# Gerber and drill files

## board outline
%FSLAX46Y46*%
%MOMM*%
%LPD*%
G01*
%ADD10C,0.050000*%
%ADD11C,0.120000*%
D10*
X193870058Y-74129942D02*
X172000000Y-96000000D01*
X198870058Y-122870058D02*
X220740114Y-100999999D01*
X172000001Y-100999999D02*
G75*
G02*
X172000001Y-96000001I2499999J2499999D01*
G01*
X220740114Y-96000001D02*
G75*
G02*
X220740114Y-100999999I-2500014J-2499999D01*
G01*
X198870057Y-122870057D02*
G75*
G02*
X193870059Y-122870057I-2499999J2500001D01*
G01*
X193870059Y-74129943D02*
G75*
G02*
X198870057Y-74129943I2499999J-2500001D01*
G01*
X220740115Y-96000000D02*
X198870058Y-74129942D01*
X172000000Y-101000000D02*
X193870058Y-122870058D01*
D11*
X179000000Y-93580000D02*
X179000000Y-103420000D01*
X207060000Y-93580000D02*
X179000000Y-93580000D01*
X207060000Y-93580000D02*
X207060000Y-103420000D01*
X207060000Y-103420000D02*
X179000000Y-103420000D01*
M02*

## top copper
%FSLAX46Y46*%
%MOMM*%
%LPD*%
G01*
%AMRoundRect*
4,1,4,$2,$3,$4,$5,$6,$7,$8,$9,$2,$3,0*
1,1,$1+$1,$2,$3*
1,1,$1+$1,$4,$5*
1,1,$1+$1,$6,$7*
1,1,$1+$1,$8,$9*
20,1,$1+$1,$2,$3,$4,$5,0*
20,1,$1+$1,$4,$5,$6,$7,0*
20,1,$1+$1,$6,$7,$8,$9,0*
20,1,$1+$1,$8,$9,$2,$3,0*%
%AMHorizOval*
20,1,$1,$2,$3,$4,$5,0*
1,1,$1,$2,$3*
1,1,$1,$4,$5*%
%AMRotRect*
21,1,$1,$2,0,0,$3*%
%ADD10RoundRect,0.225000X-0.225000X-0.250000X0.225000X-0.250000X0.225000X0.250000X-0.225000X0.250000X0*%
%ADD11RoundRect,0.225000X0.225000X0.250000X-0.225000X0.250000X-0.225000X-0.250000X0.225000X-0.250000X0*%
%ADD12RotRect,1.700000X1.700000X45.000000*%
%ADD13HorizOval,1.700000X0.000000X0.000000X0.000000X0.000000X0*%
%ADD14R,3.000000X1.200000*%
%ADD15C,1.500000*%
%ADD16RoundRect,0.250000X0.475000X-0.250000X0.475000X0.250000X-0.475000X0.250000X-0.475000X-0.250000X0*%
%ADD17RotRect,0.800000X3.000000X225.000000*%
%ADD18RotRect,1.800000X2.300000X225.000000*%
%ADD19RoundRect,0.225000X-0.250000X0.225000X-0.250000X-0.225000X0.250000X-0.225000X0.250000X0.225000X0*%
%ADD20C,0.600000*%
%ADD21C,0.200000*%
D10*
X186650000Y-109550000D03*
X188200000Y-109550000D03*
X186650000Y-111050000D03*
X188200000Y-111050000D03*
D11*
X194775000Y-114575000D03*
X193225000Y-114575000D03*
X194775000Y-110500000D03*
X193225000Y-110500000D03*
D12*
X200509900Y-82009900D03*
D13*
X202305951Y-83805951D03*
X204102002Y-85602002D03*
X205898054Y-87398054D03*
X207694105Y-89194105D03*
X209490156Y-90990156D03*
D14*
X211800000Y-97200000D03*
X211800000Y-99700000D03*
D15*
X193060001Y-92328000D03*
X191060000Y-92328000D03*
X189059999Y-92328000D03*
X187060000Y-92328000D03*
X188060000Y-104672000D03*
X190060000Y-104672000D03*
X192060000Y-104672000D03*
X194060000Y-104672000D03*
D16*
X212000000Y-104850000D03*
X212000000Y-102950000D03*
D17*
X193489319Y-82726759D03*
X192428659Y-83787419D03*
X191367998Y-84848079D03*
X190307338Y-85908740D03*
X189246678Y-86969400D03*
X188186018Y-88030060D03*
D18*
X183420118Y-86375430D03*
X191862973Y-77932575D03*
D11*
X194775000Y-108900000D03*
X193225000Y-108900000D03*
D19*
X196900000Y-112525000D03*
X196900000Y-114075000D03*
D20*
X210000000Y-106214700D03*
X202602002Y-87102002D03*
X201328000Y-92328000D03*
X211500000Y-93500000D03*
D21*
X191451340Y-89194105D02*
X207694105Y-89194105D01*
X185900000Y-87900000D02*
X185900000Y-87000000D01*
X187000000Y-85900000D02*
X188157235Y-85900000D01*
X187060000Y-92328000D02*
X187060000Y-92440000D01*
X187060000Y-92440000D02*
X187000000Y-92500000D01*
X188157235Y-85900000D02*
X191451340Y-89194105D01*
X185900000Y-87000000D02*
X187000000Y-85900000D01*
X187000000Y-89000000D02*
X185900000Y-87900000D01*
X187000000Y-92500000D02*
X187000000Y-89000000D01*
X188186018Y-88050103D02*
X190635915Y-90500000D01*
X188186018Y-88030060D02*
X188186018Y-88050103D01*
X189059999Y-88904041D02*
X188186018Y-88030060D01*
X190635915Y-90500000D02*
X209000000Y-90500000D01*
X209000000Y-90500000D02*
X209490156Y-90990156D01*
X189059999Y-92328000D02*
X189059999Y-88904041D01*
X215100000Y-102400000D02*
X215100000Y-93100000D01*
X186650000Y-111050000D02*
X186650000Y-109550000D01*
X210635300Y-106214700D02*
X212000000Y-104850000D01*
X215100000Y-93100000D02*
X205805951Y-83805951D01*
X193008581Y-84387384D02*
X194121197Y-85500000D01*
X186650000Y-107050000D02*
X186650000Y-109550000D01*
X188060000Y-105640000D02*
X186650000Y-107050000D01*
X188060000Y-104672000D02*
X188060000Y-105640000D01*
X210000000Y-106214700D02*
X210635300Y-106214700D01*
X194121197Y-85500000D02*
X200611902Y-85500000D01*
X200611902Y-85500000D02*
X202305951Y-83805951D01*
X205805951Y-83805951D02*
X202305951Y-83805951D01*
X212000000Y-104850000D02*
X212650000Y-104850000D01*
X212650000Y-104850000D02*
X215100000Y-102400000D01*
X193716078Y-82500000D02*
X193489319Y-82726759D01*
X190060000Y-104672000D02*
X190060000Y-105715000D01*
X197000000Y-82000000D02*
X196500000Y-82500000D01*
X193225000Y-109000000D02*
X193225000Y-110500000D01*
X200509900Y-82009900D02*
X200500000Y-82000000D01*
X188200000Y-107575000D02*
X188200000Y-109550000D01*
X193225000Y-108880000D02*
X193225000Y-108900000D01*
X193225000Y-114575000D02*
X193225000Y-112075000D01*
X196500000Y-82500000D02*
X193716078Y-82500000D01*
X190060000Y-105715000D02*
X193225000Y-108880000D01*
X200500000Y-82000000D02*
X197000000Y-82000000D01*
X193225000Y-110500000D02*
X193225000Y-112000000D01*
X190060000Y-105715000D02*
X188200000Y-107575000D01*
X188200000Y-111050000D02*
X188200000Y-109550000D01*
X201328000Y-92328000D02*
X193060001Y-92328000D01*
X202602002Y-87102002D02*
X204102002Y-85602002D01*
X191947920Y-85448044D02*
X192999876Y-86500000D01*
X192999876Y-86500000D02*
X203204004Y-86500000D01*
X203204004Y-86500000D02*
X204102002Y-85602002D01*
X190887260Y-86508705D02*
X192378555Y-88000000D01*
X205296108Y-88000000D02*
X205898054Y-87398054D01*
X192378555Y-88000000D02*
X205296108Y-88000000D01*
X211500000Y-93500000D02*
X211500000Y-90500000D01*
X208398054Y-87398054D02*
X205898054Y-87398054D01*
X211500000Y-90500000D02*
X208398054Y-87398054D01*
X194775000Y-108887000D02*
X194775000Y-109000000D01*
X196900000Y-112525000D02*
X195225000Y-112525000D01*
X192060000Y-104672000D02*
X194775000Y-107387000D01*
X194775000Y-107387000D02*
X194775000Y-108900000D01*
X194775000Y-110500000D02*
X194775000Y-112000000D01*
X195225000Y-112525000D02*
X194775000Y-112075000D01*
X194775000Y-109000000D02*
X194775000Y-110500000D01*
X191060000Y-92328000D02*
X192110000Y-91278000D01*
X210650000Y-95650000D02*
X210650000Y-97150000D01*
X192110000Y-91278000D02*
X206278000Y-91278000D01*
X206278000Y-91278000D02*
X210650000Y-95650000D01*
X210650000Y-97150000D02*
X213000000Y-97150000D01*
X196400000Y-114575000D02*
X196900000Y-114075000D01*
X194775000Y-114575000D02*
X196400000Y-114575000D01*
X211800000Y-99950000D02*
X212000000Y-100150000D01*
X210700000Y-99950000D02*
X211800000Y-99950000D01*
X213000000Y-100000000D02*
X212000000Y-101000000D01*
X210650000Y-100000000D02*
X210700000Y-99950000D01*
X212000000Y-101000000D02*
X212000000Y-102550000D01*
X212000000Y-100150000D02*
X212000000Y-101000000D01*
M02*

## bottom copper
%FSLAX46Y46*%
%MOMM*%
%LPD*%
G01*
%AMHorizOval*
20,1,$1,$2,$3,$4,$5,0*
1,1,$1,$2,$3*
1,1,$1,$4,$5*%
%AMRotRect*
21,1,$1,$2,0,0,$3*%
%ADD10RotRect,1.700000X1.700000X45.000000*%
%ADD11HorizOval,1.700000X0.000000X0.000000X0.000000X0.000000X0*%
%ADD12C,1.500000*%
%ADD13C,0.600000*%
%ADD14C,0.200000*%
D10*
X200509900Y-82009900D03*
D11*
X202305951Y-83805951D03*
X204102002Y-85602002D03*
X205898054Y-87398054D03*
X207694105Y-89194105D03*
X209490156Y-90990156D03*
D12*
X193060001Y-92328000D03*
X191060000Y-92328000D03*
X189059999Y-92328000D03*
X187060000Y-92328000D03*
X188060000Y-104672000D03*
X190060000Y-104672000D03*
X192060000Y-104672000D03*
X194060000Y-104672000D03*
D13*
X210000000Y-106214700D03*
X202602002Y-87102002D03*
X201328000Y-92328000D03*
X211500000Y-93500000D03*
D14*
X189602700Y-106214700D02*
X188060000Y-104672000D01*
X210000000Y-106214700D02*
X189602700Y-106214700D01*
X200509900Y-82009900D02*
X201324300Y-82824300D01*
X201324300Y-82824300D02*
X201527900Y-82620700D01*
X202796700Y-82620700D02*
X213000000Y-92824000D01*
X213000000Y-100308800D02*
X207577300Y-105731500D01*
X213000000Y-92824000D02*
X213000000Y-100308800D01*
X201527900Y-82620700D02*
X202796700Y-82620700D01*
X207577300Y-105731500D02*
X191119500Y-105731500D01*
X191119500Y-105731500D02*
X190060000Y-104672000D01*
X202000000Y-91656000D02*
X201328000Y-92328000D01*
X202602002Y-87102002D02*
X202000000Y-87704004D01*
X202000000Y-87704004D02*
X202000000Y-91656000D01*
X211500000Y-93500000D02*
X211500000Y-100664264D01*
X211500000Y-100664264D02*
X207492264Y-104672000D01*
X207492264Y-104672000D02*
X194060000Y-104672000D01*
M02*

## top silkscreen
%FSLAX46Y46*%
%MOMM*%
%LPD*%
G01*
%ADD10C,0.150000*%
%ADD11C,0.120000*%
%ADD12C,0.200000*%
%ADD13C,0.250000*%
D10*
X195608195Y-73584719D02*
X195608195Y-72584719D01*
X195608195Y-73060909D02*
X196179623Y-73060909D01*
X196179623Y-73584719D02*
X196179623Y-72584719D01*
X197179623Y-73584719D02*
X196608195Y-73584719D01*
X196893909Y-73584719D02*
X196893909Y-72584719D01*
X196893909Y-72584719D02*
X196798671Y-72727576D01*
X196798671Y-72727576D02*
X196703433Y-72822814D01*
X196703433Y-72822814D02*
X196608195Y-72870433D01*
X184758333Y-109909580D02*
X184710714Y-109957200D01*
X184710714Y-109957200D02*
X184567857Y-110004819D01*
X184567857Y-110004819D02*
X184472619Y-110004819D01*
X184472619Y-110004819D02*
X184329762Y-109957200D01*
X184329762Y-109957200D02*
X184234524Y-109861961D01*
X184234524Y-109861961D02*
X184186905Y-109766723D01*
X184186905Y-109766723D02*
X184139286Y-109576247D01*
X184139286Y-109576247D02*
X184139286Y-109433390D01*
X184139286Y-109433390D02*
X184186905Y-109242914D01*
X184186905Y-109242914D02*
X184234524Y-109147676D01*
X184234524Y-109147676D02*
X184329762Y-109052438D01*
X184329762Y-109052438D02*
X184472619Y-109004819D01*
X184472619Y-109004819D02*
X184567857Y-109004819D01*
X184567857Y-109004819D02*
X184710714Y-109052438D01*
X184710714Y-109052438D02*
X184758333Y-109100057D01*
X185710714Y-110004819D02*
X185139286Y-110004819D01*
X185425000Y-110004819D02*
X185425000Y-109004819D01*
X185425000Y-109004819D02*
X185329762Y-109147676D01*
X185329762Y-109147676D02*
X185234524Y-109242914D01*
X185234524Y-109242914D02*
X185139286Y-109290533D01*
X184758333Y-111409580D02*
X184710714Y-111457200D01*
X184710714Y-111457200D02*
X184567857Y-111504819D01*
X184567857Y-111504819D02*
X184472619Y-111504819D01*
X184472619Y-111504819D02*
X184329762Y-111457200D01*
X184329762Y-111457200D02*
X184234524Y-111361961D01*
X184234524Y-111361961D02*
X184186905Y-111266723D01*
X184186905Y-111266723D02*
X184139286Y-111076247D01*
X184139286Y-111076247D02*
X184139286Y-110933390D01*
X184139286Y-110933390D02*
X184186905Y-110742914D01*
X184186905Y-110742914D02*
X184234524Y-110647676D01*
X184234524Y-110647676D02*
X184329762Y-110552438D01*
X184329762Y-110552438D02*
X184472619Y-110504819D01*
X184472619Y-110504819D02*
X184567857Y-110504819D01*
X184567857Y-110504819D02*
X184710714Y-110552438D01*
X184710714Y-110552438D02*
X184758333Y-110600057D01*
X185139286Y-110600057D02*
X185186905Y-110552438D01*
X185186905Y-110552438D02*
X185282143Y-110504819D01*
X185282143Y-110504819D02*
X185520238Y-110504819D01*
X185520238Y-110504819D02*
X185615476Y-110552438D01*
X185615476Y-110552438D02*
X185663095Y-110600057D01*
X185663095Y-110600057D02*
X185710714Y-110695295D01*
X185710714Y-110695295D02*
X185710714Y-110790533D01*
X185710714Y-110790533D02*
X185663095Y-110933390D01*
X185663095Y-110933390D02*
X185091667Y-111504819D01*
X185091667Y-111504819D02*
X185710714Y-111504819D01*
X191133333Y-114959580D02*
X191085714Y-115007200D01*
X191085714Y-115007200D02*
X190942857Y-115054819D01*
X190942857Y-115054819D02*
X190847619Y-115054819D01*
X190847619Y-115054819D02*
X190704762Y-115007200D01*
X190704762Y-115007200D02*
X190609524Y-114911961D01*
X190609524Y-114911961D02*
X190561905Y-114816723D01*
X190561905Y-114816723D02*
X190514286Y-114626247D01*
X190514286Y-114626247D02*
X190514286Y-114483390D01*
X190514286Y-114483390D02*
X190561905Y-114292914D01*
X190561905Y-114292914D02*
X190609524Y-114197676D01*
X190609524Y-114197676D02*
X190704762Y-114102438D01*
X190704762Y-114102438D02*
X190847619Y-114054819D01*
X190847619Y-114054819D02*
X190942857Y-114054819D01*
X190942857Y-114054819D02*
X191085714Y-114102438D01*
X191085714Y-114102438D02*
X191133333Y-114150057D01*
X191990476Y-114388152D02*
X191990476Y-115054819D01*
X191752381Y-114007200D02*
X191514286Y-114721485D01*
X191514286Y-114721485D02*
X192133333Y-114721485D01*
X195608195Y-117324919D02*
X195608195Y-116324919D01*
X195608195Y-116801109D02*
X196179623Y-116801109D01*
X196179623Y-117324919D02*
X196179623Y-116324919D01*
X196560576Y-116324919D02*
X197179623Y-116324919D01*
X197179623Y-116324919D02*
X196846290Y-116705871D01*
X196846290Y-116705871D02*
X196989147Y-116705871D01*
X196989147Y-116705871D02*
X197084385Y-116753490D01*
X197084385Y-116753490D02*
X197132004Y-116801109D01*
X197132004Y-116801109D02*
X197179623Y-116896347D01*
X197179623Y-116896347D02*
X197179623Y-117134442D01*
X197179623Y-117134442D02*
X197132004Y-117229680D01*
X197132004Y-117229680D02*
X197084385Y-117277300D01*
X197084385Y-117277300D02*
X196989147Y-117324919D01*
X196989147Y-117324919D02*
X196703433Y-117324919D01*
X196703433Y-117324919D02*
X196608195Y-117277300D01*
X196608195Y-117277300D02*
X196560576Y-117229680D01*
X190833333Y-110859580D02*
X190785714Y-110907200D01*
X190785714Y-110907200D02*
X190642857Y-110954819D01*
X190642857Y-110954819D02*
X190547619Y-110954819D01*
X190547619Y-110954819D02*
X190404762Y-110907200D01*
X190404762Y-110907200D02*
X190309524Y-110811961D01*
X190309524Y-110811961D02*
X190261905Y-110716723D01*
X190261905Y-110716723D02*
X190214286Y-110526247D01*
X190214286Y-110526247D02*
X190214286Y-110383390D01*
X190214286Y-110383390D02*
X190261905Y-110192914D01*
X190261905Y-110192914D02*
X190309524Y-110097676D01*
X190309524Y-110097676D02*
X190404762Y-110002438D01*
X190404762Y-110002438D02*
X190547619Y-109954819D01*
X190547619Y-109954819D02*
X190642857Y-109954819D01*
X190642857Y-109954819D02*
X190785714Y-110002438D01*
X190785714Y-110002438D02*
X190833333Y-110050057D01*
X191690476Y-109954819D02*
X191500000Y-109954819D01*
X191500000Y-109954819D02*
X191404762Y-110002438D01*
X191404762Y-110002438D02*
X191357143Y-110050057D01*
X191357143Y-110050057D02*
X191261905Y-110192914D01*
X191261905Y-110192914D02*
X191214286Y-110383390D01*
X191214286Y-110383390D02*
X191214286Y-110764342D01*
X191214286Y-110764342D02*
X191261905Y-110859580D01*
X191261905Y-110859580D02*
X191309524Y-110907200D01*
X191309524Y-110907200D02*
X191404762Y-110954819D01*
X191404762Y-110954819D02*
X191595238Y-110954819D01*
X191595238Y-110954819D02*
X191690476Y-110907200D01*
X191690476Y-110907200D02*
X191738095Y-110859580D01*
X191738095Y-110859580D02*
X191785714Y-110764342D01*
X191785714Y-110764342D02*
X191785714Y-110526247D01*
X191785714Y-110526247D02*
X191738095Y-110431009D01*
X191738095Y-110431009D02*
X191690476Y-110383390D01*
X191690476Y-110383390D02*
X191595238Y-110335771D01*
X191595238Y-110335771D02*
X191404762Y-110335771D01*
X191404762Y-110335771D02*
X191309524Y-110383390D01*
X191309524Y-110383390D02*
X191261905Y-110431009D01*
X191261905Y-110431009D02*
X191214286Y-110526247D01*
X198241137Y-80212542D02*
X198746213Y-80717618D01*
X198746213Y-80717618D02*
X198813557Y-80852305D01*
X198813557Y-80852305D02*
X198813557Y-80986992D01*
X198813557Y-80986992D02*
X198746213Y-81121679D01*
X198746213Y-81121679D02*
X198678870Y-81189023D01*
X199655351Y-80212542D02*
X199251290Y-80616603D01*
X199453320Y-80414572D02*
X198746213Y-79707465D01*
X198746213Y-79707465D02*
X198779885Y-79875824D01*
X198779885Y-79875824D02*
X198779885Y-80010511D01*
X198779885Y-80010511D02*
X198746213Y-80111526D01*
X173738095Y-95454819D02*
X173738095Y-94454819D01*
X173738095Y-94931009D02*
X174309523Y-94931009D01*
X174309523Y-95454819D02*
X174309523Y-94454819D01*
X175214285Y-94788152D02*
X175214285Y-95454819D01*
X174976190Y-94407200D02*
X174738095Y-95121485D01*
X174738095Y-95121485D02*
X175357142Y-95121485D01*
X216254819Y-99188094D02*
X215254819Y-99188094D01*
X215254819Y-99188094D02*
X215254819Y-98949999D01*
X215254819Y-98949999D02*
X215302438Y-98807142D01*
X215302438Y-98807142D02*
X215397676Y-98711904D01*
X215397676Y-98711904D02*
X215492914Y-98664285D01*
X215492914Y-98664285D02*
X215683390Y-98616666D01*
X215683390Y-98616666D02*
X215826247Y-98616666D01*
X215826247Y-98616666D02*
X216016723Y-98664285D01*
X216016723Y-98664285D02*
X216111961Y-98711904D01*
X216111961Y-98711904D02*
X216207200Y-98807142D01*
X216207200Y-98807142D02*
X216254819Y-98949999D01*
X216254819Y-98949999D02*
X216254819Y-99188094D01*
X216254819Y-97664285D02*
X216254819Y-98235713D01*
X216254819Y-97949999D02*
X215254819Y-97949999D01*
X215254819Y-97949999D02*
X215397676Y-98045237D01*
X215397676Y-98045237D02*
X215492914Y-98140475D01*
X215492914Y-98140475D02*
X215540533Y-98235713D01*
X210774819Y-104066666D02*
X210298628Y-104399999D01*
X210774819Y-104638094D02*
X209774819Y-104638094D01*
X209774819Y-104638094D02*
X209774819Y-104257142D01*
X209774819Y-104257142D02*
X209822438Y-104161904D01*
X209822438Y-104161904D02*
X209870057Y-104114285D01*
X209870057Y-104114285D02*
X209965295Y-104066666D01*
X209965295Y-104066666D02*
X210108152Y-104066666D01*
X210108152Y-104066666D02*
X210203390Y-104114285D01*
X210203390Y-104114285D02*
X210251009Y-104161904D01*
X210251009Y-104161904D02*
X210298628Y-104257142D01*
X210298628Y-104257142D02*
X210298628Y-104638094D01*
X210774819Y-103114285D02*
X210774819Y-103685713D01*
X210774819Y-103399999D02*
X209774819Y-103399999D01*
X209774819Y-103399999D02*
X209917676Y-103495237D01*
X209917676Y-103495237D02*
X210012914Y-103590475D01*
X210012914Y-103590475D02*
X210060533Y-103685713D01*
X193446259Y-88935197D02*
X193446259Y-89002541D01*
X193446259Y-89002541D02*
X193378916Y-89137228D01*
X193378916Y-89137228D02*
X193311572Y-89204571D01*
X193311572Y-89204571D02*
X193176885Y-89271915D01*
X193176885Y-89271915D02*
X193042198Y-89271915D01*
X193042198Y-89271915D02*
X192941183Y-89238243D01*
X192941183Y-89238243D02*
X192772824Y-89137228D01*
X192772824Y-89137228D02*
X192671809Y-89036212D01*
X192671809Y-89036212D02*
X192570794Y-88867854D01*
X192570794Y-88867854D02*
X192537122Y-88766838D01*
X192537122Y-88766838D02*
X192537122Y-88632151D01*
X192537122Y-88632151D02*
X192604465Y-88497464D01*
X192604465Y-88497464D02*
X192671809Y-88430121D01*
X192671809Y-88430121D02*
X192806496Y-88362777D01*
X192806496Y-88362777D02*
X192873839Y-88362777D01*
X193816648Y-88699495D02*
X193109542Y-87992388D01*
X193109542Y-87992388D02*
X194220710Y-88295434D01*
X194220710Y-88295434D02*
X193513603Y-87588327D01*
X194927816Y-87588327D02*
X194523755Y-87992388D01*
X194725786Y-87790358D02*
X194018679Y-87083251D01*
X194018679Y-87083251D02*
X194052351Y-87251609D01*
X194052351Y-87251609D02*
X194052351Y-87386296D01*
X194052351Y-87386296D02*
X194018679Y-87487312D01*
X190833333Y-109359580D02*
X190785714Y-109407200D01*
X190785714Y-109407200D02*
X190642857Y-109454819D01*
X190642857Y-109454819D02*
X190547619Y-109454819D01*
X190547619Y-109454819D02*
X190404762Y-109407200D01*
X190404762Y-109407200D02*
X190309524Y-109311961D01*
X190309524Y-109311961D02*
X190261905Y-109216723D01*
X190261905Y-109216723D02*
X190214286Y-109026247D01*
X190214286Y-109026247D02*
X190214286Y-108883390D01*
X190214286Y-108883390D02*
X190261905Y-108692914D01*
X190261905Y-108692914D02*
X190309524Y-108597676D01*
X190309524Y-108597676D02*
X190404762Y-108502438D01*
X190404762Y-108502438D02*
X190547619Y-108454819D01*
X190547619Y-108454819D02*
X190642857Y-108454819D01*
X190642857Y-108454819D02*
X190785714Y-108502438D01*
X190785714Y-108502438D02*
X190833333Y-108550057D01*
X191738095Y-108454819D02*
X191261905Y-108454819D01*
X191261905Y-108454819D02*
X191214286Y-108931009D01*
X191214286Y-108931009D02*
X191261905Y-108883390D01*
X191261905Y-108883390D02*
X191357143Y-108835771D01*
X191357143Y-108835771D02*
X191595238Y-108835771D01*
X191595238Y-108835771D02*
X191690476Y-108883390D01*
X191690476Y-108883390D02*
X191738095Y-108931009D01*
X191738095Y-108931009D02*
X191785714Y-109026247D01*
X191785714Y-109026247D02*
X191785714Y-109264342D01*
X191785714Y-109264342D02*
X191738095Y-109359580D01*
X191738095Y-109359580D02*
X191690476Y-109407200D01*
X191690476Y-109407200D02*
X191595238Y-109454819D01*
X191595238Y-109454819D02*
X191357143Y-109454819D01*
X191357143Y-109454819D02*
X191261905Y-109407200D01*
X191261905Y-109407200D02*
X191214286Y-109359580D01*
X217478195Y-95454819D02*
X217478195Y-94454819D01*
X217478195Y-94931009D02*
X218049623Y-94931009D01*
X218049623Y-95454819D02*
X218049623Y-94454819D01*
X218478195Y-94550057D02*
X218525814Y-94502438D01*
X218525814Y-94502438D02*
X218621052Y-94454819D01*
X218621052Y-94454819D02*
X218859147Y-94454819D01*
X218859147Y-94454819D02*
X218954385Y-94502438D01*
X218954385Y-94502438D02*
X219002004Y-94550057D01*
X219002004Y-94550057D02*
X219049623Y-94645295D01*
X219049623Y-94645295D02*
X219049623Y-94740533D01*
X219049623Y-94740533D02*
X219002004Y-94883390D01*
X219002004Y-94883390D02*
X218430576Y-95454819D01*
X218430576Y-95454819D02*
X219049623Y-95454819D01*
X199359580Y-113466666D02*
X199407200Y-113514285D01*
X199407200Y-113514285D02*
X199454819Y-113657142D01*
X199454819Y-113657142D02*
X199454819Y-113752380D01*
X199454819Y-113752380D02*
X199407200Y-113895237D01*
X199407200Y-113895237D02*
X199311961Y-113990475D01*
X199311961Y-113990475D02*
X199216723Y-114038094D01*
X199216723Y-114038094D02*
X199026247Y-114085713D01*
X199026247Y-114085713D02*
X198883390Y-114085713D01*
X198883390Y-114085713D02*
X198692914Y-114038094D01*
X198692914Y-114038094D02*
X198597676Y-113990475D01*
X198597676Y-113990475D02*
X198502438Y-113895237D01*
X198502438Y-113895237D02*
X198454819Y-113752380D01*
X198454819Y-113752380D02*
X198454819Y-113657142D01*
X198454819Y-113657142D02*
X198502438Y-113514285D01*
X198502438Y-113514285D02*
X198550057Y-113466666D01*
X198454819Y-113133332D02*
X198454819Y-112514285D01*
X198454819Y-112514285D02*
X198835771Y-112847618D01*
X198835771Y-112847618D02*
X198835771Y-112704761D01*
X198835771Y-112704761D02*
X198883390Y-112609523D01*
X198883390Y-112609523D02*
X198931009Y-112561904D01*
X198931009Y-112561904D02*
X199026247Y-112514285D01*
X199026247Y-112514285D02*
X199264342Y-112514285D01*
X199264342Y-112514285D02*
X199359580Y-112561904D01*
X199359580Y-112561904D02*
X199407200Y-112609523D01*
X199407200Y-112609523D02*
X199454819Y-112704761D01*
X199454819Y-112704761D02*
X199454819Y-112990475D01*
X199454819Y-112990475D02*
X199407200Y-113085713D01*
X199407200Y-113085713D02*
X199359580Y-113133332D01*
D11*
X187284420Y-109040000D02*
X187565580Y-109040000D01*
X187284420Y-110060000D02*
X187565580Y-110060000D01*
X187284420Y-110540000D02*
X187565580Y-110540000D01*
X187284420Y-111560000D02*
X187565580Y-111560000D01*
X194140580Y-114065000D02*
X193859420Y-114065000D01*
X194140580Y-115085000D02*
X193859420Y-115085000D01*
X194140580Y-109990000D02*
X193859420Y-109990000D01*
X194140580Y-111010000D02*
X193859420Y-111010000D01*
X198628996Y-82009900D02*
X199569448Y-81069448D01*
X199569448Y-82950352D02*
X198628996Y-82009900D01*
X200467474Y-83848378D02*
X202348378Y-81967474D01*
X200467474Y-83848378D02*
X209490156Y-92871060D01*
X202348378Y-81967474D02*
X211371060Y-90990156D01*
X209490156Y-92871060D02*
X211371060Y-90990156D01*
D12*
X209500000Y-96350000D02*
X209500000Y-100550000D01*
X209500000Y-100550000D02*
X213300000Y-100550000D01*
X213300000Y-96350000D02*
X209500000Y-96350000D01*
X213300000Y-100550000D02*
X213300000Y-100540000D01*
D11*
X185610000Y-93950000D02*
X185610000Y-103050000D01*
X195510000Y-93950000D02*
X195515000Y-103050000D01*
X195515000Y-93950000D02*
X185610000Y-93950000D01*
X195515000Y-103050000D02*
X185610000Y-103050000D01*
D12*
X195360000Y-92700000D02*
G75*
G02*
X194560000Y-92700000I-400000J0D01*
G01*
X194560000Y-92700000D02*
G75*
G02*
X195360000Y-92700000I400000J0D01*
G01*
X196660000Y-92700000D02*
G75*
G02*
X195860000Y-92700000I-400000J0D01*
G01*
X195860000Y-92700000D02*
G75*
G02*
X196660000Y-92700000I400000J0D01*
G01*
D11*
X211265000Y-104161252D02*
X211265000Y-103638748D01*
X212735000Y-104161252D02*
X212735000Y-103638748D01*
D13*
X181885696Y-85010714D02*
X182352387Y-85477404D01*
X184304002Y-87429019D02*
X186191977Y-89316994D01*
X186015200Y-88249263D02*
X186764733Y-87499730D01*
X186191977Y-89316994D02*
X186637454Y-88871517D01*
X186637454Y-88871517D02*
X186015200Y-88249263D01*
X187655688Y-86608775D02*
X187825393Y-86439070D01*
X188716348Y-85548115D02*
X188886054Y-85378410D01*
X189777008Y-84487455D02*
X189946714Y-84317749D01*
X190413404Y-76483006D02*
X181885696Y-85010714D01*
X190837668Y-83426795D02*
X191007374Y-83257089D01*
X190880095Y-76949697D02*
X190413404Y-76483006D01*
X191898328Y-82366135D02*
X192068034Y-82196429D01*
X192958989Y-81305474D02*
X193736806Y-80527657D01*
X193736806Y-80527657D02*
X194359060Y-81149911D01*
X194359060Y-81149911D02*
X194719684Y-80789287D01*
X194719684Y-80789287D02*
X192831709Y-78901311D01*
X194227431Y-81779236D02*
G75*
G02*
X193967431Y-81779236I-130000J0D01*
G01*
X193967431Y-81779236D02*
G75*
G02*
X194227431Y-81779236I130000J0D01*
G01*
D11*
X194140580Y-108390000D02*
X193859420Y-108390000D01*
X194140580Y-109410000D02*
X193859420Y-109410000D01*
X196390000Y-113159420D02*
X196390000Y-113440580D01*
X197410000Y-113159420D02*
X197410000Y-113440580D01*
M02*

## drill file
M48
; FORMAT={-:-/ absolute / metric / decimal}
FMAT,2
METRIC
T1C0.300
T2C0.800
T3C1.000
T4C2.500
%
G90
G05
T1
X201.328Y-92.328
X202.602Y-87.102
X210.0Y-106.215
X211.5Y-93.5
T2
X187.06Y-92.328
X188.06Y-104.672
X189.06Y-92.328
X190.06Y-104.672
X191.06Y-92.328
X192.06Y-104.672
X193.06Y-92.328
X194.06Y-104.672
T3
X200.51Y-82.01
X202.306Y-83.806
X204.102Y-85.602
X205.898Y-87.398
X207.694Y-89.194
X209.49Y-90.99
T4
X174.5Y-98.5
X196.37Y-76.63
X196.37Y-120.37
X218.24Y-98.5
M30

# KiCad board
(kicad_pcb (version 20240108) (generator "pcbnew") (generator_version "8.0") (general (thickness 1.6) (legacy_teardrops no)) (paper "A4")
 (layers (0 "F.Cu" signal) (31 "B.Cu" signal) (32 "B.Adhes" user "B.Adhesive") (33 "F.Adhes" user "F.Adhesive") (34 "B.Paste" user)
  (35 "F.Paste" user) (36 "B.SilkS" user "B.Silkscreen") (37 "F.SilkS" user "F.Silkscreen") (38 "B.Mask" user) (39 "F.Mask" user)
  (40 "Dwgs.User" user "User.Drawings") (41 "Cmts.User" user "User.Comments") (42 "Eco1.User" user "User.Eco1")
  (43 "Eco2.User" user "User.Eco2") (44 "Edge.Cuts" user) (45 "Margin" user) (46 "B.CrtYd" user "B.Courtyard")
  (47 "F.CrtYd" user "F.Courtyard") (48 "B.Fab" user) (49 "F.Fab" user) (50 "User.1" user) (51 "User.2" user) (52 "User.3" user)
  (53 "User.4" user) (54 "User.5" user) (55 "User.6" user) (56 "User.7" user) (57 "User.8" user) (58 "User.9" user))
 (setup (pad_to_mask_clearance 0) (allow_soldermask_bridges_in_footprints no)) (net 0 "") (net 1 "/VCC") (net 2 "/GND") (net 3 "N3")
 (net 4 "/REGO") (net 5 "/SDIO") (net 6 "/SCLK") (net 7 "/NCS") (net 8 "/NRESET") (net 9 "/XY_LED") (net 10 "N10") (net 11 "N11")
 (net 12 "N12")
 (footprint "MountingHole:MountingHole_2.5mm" (layer "F.Cu") (at 196.3701 76.6299)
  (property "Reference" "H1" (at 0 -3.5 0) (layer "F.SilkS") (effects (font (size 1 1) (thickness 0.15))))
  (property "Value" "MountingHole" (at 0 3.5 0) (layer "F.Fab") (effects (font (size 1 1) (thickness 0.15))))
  (pad "" np_thru_hole circle (at 0 0) (size 2.5 2.5) (drill 2.5) (layers "*.Cu" "*.Mask")))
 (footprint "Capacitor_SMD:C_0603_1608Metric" (layer "F.Cu") (at 187.425 109.55)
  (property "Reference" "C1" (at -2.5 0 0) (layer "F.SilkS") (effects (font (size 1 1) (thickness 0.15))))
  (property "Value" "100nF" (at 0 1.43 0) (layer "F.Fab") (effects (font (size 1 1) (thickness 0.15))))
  (fp_line (start -0.14058 -0.51) (end 0.14058 -0.51) (stroke (width 0.12) (type solid)) (layer "F.SilkS"))
  (fp_line (start -0.14058 0.51) (end 0.14058 0.51) (stroke (width 0.12) (type solid)) (layer "F.SilkS"))
  (pad "1" smd roundrect (at -0.775 0) (size 0.9 0.95) (layers "F.Cu" "F.Paste" "F.Mask") (roundrect_rratio 0.25) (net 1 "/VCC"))
  (pad "2" smd roundrect (at 0.775 0) (size 0.9 0.95) (layers "F.Cu" "F.Paste" "F.Mask") (roundrect_rratio 0.25) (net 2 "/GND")))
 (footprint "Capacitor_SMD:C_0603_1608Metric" (layer "F.Cu") (at 187.425 111.05)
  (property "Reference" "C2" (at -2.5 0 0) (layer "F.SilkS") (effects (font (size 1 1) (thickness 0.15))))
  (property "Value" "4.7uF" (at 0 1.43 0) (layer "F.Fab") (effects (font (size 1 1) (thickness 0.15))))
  (fp_line (start -0.14058 -0.51) (end 0.14058 -0.51) (stroke (width 0.12) (type solid)) (layer "F.SilkS"))
  (fp_line (start -0.14058 0.51) (end 0.14058 0.51) (stroke (width 0.12) (type solid)) (layer "F.SilkS"))
  (pad "1" smd roundrect (at -0.775 0) (size 0.9 0.95) (layers "F.Cu" "F.Paste" "F.Mask") (roundrect_rratio 0.25) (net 1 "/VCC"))
  (pad "2" smd roundrect (at 0.775 0) (size 0.9 0.95) (layers "F.Cu" "F.Paste" "F.Mask") (roundrect_rratio 0.25) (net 2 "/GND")))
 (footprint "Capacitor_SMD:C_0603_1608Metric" (layer "F.Cu") (at 194 114.575 180)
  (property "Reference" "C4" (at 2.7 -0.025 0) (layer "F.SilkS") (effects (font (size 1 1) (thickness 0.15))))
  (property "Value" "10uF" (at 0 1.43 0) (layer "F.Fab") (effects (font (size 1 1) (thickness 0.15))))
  (fp_line (start -0.14058 0.51) (end 0.14058 0.51) (stroke (width 0.12) (type solid)) (layer "F.SilkS"))
  (fp_line (start -0.14058 -0.51) (end 0.14058 -0.51) (stroke (width 0.12) (type solid)) (layer "F.SilkS"))
  (pad "1" smd roundrect (at -0.775 0 180) (size 0.9 0.95) (layers "F.Cu" "F.Paste" "F.Mask") (roundrect_rratio 0.25) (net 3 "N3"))
  (pad "2" smd roundrect (at 0.775 0 180) (size 0.9 0.95) (layers "F.Cu" "F.Paste" "F.Mask") (roundrect_rratio 0.25) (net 2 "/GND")))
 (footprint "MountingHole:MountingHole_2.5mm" (layer "F.Cu") (at 196.3701 120.3701)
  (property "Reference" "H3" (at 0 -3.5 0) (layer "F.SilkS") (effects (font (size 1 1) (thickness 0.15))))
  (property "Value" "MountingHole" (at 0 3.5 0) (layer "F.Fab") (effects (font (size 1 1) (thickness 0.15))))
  (pad "" np_thru_hole circle (at 0 0) (size 2.5 2.5) (drill 2.5) (layers "*.Cu" "*.Mask")))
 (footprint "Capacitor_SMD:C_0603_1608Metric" (layer "F.Cu") (at 194 110.5 180)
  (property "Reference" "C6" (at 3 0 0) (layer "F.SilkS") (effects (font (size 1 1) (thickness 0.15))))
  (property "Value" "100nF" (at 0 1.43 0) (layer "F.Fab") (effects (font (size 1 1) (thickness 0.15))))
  (fp_line (start -0.14058 0.51) (end 0.14058 0.51) (stroke (width 0.12) (type solid)) (layer "F.SilkS"))
  (fp_line (start -0.14058 -0.51) (end 0.14058 -0.51) (stroke (width 0.12) (type solid)) (layer "F.SilkS"))
  (pad "1" smd roundrect (at -0.775 0 180) (size 0.9 0.95) (layers "F.Cu" "F.Paste" "F.Mask") (roundrect_rratio 0.25) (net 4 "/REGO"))
  (pad "2" smd roundrect (at 0.775 0 180) (size 0.9 0.95) (layers "F.Cu" "F.Paste" "F.Mask") (roundrect_rratio 0.25) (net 2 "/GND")))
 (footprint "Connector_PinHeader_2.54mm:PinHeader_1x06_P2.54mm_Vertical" (layer "F.Cu") (at 200.5099 82.0099 45)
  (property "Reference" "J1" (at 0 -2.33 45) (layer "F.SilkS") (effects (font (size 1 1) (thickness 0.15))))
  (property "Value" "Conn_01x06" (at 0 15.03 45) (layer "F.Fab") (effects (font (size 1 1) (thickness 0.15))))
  (fp_line (start -1.33 -1.33) (end 0 -1.33) (stroke (width 0.12) (type solid)) (layer "F.SilkS"))
  (fp_line (start -1.33 0) (end -1.33 -1.33) (stroke (width 0.12) (type solid)) (layer "F.SilkS"))
  (fp_line (start -1.33 1.270001) (end 1.33 1.270001) (stroke (width 0.12) (type solid)) (layer "F.SilkS"))
  (fp_line (start -1.33 1.270001) (end -1.33 14.03) (stroke (width 0.12) (type solid)) (layer "F.SilkS"))
  (fp_line (start 1.33 1.270001) (end 1.33 14.03) (stroke (width 0.12) (type solid)) (layer "F.SilkS"))
  (fp_line (start -1.33 14.03) (end 1.33 14.03) (stroke (width 0.12) (type solid)) (layer "F.SilkS"))
  (pad "1" thru_hole rect (at 0 0 45) (size 1.7 1.7) (drill 1) (layers "*.Cu" "*.Mask") (remove_unused_layers no) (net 2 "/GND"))
  (pad "2" thru_hole oval (at 0 2.54 45) (size 1.7 1.7) (drill 1) (layers "*.Cu" "*.Mask") (remove_unused_layers no) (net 1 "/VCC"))
  (pad "3" thru_hole oval (at 0 5.079999 45) (size 1.7 1.7) (drill 1) (layers "*.Cu" "*.Mask") (remove_unused_layers no) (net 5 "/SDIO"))
  (pad "4" thru_hole oval (at 0 7.62 45) (size 1.7 1.7) (drill 1) (layers "*.Cu" "*.Mask") (remove_unused_layers no) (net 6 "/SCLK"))
  (pad "5" thru_hole oval (at 0 10.16 45) (size 1.7 1.7) (drill 1) (layers "*.Cu" "*.Mask") (remove_unused_layers no) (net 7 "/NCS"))
  (pad "6" thru_hole oval (at 0 12.7 45) (size 1.7 1.7) (drill 1) (layers "*.Cu" "*.Mask") (remove_unused_layers no) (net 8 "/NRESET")))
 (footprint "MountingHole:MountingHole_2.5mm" (layer "F.Cu") (at 174.5 98.5)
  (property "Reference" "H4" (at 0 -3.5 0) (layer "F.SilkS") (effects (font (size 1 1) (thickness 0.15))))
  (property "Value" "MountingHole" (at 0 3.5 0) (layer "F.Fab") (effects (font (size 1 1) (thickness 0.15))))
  (pad "" np_thru_hole circle (at 0 0) (size 2.5 2.5) (drill 2.5) (layers "*.Cu" "*.Mask")))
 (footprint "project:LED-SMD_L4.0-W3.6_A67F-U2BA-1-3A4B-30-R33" (layer "F.Cu") (at 211.8 98.45 -90)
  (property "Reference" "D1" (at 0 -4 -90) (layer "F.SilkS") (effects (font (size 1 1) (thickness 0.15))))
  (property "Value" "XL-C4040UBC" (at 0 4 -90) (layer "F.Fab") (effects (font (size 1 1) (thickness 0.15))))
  (fp_line (start -2.1 2.3) (end 2.1 2.3) (stroke (width 0.2) (type solid)) (layer "F.SilkS"))
  (fp_line (start 2.1 2.3) (end 2.1 -1.5) (stroke (width 0.2) (type solid)) (layer "F.SilkS"))
  (fp_line (start -2.1 -1.5) (end -2.1 2.3) (stroke (width 0.2) (type solid)) (layer "F.SilkS"))
  (fp_line (start 2.1 -1.5) (end 2.09 -1.5) (stroke (width 0.2) (type solid)) (layer "F.SilkS"))
  (pad "1" smd rect (at -1.25 0 270) (size 1.2 3) (layers "F.Cu" "F.Paste" "F.Mask") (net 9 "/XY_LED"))
  (pad "2" smd rect (at 1.25 0 270) (size 1.2 3) (layers "F.Cu" "F.Paste" "F.Mask") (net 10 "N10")))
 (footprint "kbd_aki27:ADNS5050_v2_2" (layer "F.Cu") (at 191.06 98.5)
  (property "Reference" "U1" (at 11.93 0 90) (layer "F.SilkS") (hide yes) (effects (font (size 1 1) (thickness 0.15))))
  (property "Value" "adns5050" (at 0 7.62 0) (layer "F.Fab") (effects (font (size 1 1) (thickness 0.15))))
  (fp_line (start -5.45 -4.55) (end -5.45 4.55) (stroke (width 0.12) (type solid)) (layer "F.SilkS"))
  (fp_line (start 4.45 -4.55) (end 4.455 4.55) (stroke (width 0.12) (type solid)) (layer "F.SilkS"))
  (fp_line (start 4.455 -4.55) (end -5.45 -4.55) (stroke (width 0.12) (type solid)) (layer "F.SilkS"))
  (fp_line (start 4.455 4.55) (end -5.45 4.55) (stroke (width 0.12) (type solid)) (layer "F.SilkS"))
  (fp_circle (center 3.9 -5.8) (end 3.5 -5.8) (stroke (width 0.2) (type solid)) (fill none) (layer "F.SilkS"))
  (fp_circle (center 5.2 -5.8) (end 4.8 -5.8) (stroke (width 0.2) (type solid)) (fill none) (layer "F.SilkS"))
  (fp_line (start -12.06 -4.92) (end -12.06 4.92) (stroke (width 0.12) (type solid)) (layer "Edge.Cuts"))
  (fp_line (start 16 -4.92) (end -12.06 -4.92) (stroke (width 0.12) (type solid)) (layer "Edge.Cuts"))
  (fp_line (start 16 -4.92) (end 16 4.92) (stroke (width 0.12) (type solid)) (layer "Edge.Cuts"))
  (fp_line (start 16 4.92) (end -12.06 4.92) (stroke (width 0.12) (type solid)) (layer "Edge.Cuts"))
  (pad "1" thru_hole circle (at 2.000001 -6.172 180) (size 1.5 1.5) (drill 0.8) (layers "*.Cu" "*.Mask") (remove_unused_layers no)
   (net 5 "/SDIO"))
  (pad "2" thru_hole circle (at 0 -6.172 180) (size 1.5 1.5) (drill 0.8) (layers "*.Cu" "*.Mask") (remove_unused_layers no)
   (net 9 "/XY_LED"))
  (pad "3" thru_hole circle (at -2.000001 -6.172 180) (size 1.5 1.5) (drill 0.8) (layers "*.Cu" "*.Mask") (remove_unused_layers no)
   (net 8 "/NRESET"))
  (pad "4" thru_hole circle (at -4 -6.172 180) (size 1.5 1.5) (drill 0.8) (layers "*.Cu" "*.Mask") (remove_unused_layers no) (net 7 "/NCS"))
  (pad "5" thru_hole circle (at -3 6.172 180) (size 1.5 1.5) (drill 0.8) (layers "*.Cu" "*.Mask") (remove_unused_layers no) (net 1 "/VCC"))
  (pad "6" thru_hole circle (at -1 6.172 180) (size 1.5 1.5) (drill 0.8) (layers "*.Cu" "*.Mask") (remove_unused_layers no) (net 2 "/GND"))
  (pad "7" thru_hole circle (at 1 6.172 180) (size 1.5 1.5) (drill 0.8) (layers "*.Cu" "*.Mask") (remove_unused_layers no) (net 4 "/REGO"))
  (pad "8" thru_hole circle (at 3 6.172 180) (size 1.5 1.5) (drill 0.8) (layers "*.Cu" "*.Mask") (remove_unused_layers no) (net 6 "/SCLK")))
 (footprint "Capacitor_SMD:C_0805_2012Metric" (layer "F.Cu") (at 212 103.9 90)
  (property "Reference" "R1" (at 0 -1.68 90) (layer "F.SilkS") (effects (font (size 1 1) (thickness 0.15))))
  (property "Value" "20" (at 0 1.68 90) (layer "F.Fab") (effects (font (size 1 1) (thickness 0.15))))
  (fp_line (start -0.261252 -0.735) (end 0.261252 -0.735) (stroke (width 0.12) (type solid)) (layer "F.SilkS"))
  (fp_line (start -0.261252 0.735) (end 0.261252 0.735) (stroke (width 0.12) (type solid)) (layer "F.SilkS"))
  (pad "1" smd roundrect (at -0.95 0 90) (size 1 1.45) (layers "F.Cu" "F.Paste" "F.Mask") (roundrect_rratio 0.25) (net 1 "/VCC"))
  (pad "2" smd roundrect (at 0.95 0 90) (size 1 1.45) (layers "F.Cu" "F.Paste" "F.Mask") (roundrect_rratio 0.25) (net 10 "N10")))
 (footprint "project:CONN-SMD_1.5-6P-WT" (layer "F.Cu") (at 189.246678 83.759135 -135)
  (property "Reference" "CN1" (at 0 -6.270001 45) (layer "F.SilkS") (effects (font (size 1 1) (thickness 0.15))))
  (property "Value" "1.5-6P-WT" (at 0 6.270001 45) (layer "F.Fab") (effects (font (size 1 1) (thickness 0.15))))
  (fp_line (start 6.09 4.32) (end 6.09 3.66) (stroke (width 0.25) (type solid)) (layer "F.SilkS"))
  (fp_line (start 6.09 0.9) (end 6.09 -1.77) (stroke (width 0.25) (type solid)) (layer "F.SilkS"))
  (fp_line (start 5.46 -0.89) (end 4.4 -0.89) (stroke (width 0.25) (type solid)) (layer "F.SilkS"))
  (fp_line (start 6.09 -1.77) (end 5.46 -1.77) (stroke (width 0.25) (type solid)) (layer "F.SilkS"))
  (fp_line (start 5.46 -1.77) (end 5.46 -0.89) (stroke (width 0.25) (type solid)) (layer "F.SilkS"))
  (fp_line (start 3.14 -0.89) (end 2.9 -0.89) (stroke (width 0.25) (type solid)) (layer "F.SilkS"))
  (fp_line (start 1.64 -0.89) (end 1.4 -0.890001) (stroke (width 0.25) (type solid)) (layer "F.SilkS"))
  (fp_line (start 0.14 -0.89) (end -0.1 -0.89) (stroke (width 0.25) (type solid)) (layer "F.SilkS"))
  (fp_line (start -5.97 4.32) (end 6.09 4.32) (stroke (width 0.25) (type solid)) (layer "F.SilkS"))
  (fp_line (start -1.36 -0.89) (end -1.6 -0.89) (stroke (width 0.25) (type solid)) (layer "F.SilkS"))
  (fp_line (start -5.97 3.66) (end -5.97 4.32) (stroke (width 0.25) (type solid)) (layer "F.SilkS"))
  (fp_line (start -2.859999 -0.89) (end -3.1 -0.89) (stroke (width 0.25) (type solid)) (layer "F.SilkS"))
  (fp_line (start -4.360001 -0.89) (end -5.46 -0.89) (stroke (width 0.25) (type solid)) (layer "F.SilkS"))
  (fp_line (start -5.46 -0.89) (end -5.46 -1.77) (stroke (width 0.25) (type solid)) (layer "F.SilkS"))
  (fp_line (start -5.46 -1.77) (end -5.969999 -1.77) (stroke (width 0.25) (type solid)) (layer "F.SilkS"))
  (fp_line (start -5.969999 -1.77) (end -5.97 0.900001) (stroke (width 0.25) (type solid)) (layer "F.SilkS"))
  (fp_circle (center -4.83 -2.03) (end -4.7 -2.03) (stroke (width 0.25) (type solid)) (fill none) (layer "F.SilkS"))
  (pad "1" smd rect (at -3.73 -2.27 225) (size 0.8 3) (layers "F.Cu" "F.Paste" "F.Mask") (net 2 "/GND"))
  (pad "2" smd rect (at -2.230001 -2.27 225) (size 0.8 3) (layers "F.Cu" "F.Paste" "F.Mask") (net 1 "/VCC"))
  (pad "3" smd rect (at -0.73 -2.269999 225) (size 0.8 3) (layers "F.Cu" "F.Paste" "F.Mask") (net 5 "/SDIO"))
  (pad "4" smd rect (at 0.77 -2.27 225) (size 0.8 3) (layers "F.Cu" "F.Paste" "F.Mask") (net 6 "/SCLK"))
  (pad "5" smd rect (at 2.27 -2.27 225) (size 0.8 3) (layers "F.Cu" "F.Paste" "F.Mask") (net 7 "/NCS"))
  (pad "6" smd rect (at 3.77 -2.27 225) (size 0.8 3) (layers "F.Cu" "F.Paste" "F.Mask") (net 8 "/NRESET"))
  (pad "7" smd rect (at 5.97 2.27 225) (size 1.8 2.3) (layers "F.Cu" "F.Paste" "F.Mask") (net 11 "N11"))
  (pad "8" smd rect (at -5.97 2.27 225) (size 1.8 2.3) (layers "F.Cu" "F.Paste" "F.Mask") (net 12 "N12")))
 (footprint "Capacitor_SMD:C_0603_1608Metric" (layer "F.Cu") (at 194 108.9 180)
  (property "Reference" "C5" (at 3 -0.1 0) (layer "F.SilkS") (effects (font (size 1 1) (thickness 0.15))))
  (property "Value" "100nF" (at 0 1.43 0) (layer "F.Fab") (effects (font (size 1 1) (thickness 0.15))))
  (fp_line (start -0.14058 0.51) (end 0.14058 0.51) (stroke (width 0.12) (type solid)) (layer "F.SilkS"))
  (fp_line (start -0.14058 -0.51) (end 0.14058 -0.51) (stroke (width 0.12) (type solid)) (layer "F.SilkS"))
  (pad "1" smd roundrect (at -0.775 0 180) (size 0.9 0.95) (layers "F.Cu" "F.Paste" "F.Mask") (roundrect_rratio 0.25) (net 4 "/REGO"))
  (pad "2" smd roundrect (at 0.775 0 180) (size 0.9 0.95) (layers "F.Cu" "F.Paste" "F.Mask") (roundrect_rratio 0.25) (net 2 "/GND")))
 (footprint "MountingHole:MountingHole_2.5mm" (layer "F.Cu") (at 218.2401 98.5)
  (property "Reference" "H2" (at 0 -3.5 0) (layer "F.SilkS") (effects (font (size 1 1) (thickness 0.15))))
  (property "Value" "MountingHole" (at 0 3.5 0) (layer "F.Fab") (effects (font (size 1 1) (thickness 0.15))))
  (pad "" np_thru_hole circle (at 0 0) (size 2.5 2.5) (drill 2.5) (layers "*.Cu" "*.Mask")))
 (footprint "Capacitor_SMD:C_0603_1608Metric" (layer "F.Cu") (at 196.9 113.3 -90)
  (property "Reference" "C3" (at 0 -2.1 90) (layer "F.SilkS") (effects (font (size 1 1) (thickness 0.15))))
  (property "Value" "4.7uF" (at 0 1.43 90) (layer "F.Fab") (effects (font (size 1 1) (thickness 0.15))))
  (fp_line (start -0.14058 0.51) (end 0.14058 0.51) (stroke (width 0.12) (type solid)) (layer "F.SilkS"))
  (fp_line (start -0.14058 -0.51) (end 0.14058 -0.51) (stroke (width 0.12) (type solid)) (layer "F.SilkS"))
  (pad "1" smd roundrect (at -0.775 0 270) (size 0.9 0.95) (layers "F.Cu" "F.Paste" "F.Mask") (roundrect_rratio 0.25) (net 4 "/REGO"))
  (pad "2" smd roundrect (at 0.775 0 270) (size 0.9 0.95) (layers "F.Cu" "F.Paste" "F.Mask") (roundrect_rratio 0.25) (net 3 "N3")))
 (gr_line (start 193.870058 74.129942) (end 172 96) (stroke (width 0.05) (type default)) (layer "Edge.Cuts"))
 (gr_line (start 198.870058 122.870058) (end 220.740114 100.999999) (stroke (width 0.05) (type default)) (layer "Edge.Cuts"))
 (gr_arc (start 172.000001 100.999999) (mid 170.964468 98.5) (end 172.000001 96.000001) (stroke (width 0.05) (type default))
  (layer "Edge.Cuts"))
 (gr_arc (start 220.740114 96.000001) (mid 221.775647 98.5) (end 220.740114 100.999999) (stroke (width 0.05) (type default))
  (layer "Edge.Cuts"))
 (gr_arc (start 198.870057 122.870057) (mid 196.370058 123.90559) (end 193.870059 122.870057) (stroke (width 0.05) (type default))
  (layer "Edge.Cuts"))
 (gr_arc (start 193.870059 74.129943) (mid 196.370058 73.09441) (end 198.870057 74.129943) (stroke (width 0.05) (type default))
  (layer "Edge.Cuts"))
 (gr_line (start 220.740115 96) (end 198.870058 74.129942) (stroke (width 0.05) (type default)) (layer "Edge.Cuts"))
 (gr_line (start 172 101) (end 193.870058 122.870058) (stroke (width 0.05) (type default)) (layer "Edge.Cuts"))
 (segment (start 191.45134 89.194105) (end 207.694105 89.194105) (width 0.2) (layer "F.Cu") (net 7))
 (segment (start 185.9 87.9) (end 185.9 87) (width 0.2) (layer "F.Cu") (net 7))
 (segment (start 187 85.9) (end 188.157235 85.9) (width 0.2) (layer "F.Cu") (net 7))
 (segment (start 187.06 92.328) (end 187.06 92.44) (width 0.2) (layer "F.Cu") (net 7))
 (segment (start 187.06 92.44) (end 187 92.5) (width 0.2) (layer "F.Cu") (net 7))
 (segment (start 188.157235 85.9) (end 191.45134 89.194105) (width 0.2) (layer "F.Cu") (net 7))
 (segment (start 185.9 87) (end 187 85.9) (width 0.2) (layer "F.Cu") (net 7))
 (segment (start 187 89) (end 185.9 87.9) (width 0.2) (layer "F.Cu") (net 7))
 (segment (start 187 92.5) (end 187 89) (width 0.2) (layer "F.Cu") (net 7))
 (segment (start 188.186018 88.050103) (end 190.635915 90.5) (width 0.2) (layer "F.Cu") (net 8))
 (segment (start 188.186018 88.03006) (end 188.186018 88.050103) (width 0.2) (layer "F.Cu") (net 8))
 (segment (start 189.059999 88.904041) (end 188.186018 88.03006) (width 0.2) (layer "F.Cu") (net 8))
 (segment (start 190.635915 90.5) (end 209 90.5) (width 0.2) (layer "F.Cu") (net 8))
 (segment (start 209 90.5) (end 209.490156 90.990156) (width 0.2) (layer "F.Cu") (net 8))
 (segment (start 189.059999 92.328) (end 189.059999 88.904041) (width 0.2) (layer "F.Cu") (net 8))
 (segment (start 215.1 102.4) (end 215.1 93.1) (width 0.2) (layer "F.Cu") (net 1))
 (segment (start 186.65 111.05) (end 186.65 109.55) (width 0.2) (layer "F.Cu") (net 1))
 (segment (start 210.6353 106.2147) (end 212 104.85) (width 0.2) (layer "F.Cu") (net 1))
 (segment (start 215.1 93.1) (end 205.805951 83.805951) (width 0.2) (layer "F.Cu") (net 1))
 (segment (start 193.008581 84.387384) (end 194.121197 85.5) (width 0.2) (layer "F.Cu") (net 1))
 (segment (start 186.65 107.05) (end 186.65 109.55) (width 0.2) (layer "F.Cu") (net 1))
 (segment (start 188.06 105.64) (end 186.65 107.05) (width 0.2) (layer "F.Cu") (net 1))
 (segment (start 188.06 104.672) (end 188.06 105.64) (width 0.2) (layer "F.Cu") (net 1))
 (segment (start 210 106.2147) (end 210.6353 106.2147) (width 0.2) (layer "F.Cu") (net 1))
 (segment (start 194.121197 85.5) (end 200.611902 85.5) (width 0.2) (layer "F.Cu") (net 1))
 (segment (start 200.611902 85.5) (end 202.305951 83.805951) (width 0.2) (layer "F.Cu") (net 1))
 (segment (start 205.805951 83.805951) (end 202.305951 83.805951) (width 0.2) (layer "F.Cu") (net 1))
 (segment (start 212 104.85) (end 212.65 104.85) (width 0.2) (layer "F.Cu") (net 1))
 (segment (start 212.65 104.85) (end 215.1 102.4) (width 0.2) (layer "F.Cu") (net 1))
 (via (at 210 106.2147) (size 0.6) (drill 0.3) (layers "F.Cu" "B.Cu") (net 1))
 (segment (start 189.6027 106.2147) (end 188.06 104.672) (width 0.2) (layer "B.Cu") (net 1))
 (segment (start 210 106.2147) (end 189.6027 106.2147) (width 0.2) (layer "B.Cu") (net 1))
 (segment (start 193.716078 82.5) (end 193.489319 82.726759) (width 0.2) (layer "F.Cu") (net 2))
 (segment (start 190.06 104.672) (end 190.06 105.715) (width 0.2) (layer "F.Cu") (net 2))
 (segment (start 197 82) (end 196.5 82.5) (width 0.2) (layer "F.Cu") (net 2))
 (segment (start 193.225 109) (end 193.225 110.5) (width 0.2) (layer "F.Cu") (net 2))
 (segment (start 200.5099 82.0099) (end 200.5 82) (width 0.2) (layer "F.Cu") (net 2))
 (segment (start 188.2 107.575) (end 188.2 109.55) (width 0.2) (layer "F.Cu") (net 2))
 (segment (start 193.225 108.88) (end 193.225 108.9) (width 0.2) (layer "F.Cu") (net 2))
 (segment (start 193.225 114.575) (end 193.225 112.075) (width 0.2) (layer "F.Cu") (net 2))
 (segment (start 196.5 82.5) (end 193.716078 82.5) (width 0.2) (layer "F.Cu") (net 2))
 (segment (start 190.06 105.715) (end 193.225 108.88) (width 0.2) (layer "F.Cu") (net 2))
 (segment (start 200.5 82) (end 197 82) (width 0.2) (layer "F.Cu") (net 2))
 (segment (start 193.225 110.5) (end 193.225 112) (width 0.2) (layer "F.Cu") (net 2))
 (segment (start 190.06 105.715) (end 188.2 107.575) (width 0.2) (layer "F.Cu") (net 2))
 (segment (start 188.2 111.05) (end 188.2 109.55) (width 0.2) (layer "F.Cu") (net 2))
 (segment (start 200.5099 82.0099) (end 201.3243 82.8243) (width 0.2) (layer "B.Cu") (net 2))
 (segment (start 201.3243 82.8243) (end 201.5279 82.6207) (width 0.2) (layer "B.Cu") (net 2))
 (segment (start 202.7967 82.6207) (end 213 92.824) (width 0.2) (layer "B.Cu") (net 2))
 (segment (start 213 100.3088) (end 207.5773 105.7315) (width 0.2) (layer "B.Cu") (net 2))
 (segment (start 213 92.824) (end 213 100.3088) (width 0.2) (layer "B.Cu") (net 2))
 (segment (start 201.5279 82.6207) (end 202.7967 82.6207) (width 0.2) (layer "B.Cu") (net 2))
 (segment (start 207.5773 105.7315) (end 191.1195 105.7315) (width 0.2) (layer "B.Cu") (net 2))
 (segment (start 191.1195 105.7315) (end 190.06 104.672) (width 0.2) (layer "B.Cu") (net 2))
 (segment (start 201.328 92.328) (end 193.060001 92.328) (width 0.2) (layer "F.Cu") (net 5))
 (segment (start 202.602002 87.102002) (end 204.102002 85.602002) (width 0.2) (layer "F.Cu") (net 5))
 (segment (start 191.94792 85.448044) (end 192.999876 86.5) (width 0.2) (layer "F.Cu") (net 5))
 (segment (start 192.999876 86.5) (end 203.204004 86.5) (width 0.2) (layer "F.Cu") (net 5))
 (segment (start 203.204004 86.5) (end 204.102002 85.602002) (width 0.2) (layer "F.Cu") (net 5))
 (via (at 202.602002 87.102002) (size 0.6) (drill 0.3) (layers "F.Cu" "B.Cu") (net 5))
 (via (at 201.328 92.328) (size 0.6) (drill 0.3) (layers "F.Cu" "B.Cu") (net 5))
 (segment (start 202 91.656) (end 201.328 92.328) (width 0.2) (layer "B.Cu") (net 5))
 (segment (start 202.602002 87.102002) (end 202 87.704004) (width 0.2) (layer "B.Cu") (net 5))
 (segment (start 202 87.704004) (end 202 91.656) (width 0.2) (layer "B.Cu") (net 5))
 (segment (start 190.88726 86.508705) (end 192.378555 88) (width 0.2) (layer "F.Cu") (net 6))
 (segment (start 205.296108 88) (end 205.898054 87.398054) (width 0.2) (layer "F.Cu") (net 6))
 (segment (start 192.378555 88) (end 205.296108 88) (width 0.2) (layer "F.Cu") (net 6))
 (segment (start 211.5 93.5) (end 211.5 90.5) (width 0.2) (layer "F.Cu") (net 6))
 (segment (start 208.398054 87.398054) (end 205.898054 87.398054) (width 0.2) (layer "F.Cu") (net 6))
 (segment (start 211.5 90.5) (end 208.398054 87.398054) (width 0.2) (layer "F.Cu") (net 6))
 (via (at 211.5 93.5) (size 0.6) (drill 0.3) (layers "F.Cu" "B.Cu") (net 6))
 (segment (start 211.5 93.5) (end 211.5 100.664264) (width 0.2) (layer "B.Cu") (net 6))
 (segment (start 211.5 100.664264) (end 207.492264 104.672) (width 0.2) (layer "B.Cu") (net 6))
 (segment (start 207.492264 104.672) (end 194.06 104.672) (width 0.2) (layer "B.Cu") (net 6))
 (segment (start 194.775 108.887) (end 194.775 109) (width 0.2) (layer "F.Cu") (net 4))
 (segment (start 196.9 112.525) (end 195.225 112.525) (width 0.2) (layer "F.Cu") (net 4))
 (segment (start 192.06 104.672) (end 194.775 107.387) (width 0.2) (layer "F.Cu") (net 4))
 (segment (start 194.775 107.387) (end 194.775 108.9) (width 0.2) (layer "F.Cu") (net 4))
 (segment (start 194.775 110.5) (end 194.775 112) (width 0.2) (layer "F.Cu") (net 4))
 (segment (start 195.225 112.525) (end 194.775 112.075) (width 0.2) (layer "F.Cu") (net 4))
 (segment (start 194.775 109) (end 194.775 110.5) (width 0.2) (layer "F.Cu") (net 4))
 (segment (start 191.06 92.328) (end 192.11 91.278) (width 0.2) (layer "F.Cu") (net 9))
 (segment (start 210.65 95.65) (end 210.65 97.15) (width 0.2) (layer "F.Cu") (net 9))
 (segment (start 192.11 91.278) (end 206.278 91.278) (width 0.2) (layer "F.Cu") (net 9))
 (segment (start 206.278 91.278) (end 210.65 95.65) (width 0.2) (layer "F.Cu") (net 9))
 (segment (start 210.65 97.15) (end 213 97.15) (width 0.2) (layer "F.Cu") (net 9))
 (segment (start 196.4 114.575) (end 196.9 114.075) (width 0.2) (layer "F.Cu") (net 3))
 (segment (start 194.775 114.575) (end 196.4 114.575) (width 0.2) (layer "F.Cu") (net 3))
 (segment (start 211.8 99.95) (end 212 100.15) (width 0.2) (layer "F.Cu") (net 10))
 (segment (start 210.7 99.95) (end 211.8 99.95) (width 0.2) (layer "F.Cu") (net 10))
 (segment (start 213 100) (end 212 101) (width 0.2) (layer "F.Cu") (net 10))
 (segment (start 210.65 100) (end 210.7 99.95) (width 0.2) (layer "F.Cu") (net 10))
 (segment (start 212 101) (end 212 102.55) (width 0.2) (layer "F.Cu") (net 10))
 (segment (start 212 100.15) (end 212 101) (width 0.2) (layer "F.Cu") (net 10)))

